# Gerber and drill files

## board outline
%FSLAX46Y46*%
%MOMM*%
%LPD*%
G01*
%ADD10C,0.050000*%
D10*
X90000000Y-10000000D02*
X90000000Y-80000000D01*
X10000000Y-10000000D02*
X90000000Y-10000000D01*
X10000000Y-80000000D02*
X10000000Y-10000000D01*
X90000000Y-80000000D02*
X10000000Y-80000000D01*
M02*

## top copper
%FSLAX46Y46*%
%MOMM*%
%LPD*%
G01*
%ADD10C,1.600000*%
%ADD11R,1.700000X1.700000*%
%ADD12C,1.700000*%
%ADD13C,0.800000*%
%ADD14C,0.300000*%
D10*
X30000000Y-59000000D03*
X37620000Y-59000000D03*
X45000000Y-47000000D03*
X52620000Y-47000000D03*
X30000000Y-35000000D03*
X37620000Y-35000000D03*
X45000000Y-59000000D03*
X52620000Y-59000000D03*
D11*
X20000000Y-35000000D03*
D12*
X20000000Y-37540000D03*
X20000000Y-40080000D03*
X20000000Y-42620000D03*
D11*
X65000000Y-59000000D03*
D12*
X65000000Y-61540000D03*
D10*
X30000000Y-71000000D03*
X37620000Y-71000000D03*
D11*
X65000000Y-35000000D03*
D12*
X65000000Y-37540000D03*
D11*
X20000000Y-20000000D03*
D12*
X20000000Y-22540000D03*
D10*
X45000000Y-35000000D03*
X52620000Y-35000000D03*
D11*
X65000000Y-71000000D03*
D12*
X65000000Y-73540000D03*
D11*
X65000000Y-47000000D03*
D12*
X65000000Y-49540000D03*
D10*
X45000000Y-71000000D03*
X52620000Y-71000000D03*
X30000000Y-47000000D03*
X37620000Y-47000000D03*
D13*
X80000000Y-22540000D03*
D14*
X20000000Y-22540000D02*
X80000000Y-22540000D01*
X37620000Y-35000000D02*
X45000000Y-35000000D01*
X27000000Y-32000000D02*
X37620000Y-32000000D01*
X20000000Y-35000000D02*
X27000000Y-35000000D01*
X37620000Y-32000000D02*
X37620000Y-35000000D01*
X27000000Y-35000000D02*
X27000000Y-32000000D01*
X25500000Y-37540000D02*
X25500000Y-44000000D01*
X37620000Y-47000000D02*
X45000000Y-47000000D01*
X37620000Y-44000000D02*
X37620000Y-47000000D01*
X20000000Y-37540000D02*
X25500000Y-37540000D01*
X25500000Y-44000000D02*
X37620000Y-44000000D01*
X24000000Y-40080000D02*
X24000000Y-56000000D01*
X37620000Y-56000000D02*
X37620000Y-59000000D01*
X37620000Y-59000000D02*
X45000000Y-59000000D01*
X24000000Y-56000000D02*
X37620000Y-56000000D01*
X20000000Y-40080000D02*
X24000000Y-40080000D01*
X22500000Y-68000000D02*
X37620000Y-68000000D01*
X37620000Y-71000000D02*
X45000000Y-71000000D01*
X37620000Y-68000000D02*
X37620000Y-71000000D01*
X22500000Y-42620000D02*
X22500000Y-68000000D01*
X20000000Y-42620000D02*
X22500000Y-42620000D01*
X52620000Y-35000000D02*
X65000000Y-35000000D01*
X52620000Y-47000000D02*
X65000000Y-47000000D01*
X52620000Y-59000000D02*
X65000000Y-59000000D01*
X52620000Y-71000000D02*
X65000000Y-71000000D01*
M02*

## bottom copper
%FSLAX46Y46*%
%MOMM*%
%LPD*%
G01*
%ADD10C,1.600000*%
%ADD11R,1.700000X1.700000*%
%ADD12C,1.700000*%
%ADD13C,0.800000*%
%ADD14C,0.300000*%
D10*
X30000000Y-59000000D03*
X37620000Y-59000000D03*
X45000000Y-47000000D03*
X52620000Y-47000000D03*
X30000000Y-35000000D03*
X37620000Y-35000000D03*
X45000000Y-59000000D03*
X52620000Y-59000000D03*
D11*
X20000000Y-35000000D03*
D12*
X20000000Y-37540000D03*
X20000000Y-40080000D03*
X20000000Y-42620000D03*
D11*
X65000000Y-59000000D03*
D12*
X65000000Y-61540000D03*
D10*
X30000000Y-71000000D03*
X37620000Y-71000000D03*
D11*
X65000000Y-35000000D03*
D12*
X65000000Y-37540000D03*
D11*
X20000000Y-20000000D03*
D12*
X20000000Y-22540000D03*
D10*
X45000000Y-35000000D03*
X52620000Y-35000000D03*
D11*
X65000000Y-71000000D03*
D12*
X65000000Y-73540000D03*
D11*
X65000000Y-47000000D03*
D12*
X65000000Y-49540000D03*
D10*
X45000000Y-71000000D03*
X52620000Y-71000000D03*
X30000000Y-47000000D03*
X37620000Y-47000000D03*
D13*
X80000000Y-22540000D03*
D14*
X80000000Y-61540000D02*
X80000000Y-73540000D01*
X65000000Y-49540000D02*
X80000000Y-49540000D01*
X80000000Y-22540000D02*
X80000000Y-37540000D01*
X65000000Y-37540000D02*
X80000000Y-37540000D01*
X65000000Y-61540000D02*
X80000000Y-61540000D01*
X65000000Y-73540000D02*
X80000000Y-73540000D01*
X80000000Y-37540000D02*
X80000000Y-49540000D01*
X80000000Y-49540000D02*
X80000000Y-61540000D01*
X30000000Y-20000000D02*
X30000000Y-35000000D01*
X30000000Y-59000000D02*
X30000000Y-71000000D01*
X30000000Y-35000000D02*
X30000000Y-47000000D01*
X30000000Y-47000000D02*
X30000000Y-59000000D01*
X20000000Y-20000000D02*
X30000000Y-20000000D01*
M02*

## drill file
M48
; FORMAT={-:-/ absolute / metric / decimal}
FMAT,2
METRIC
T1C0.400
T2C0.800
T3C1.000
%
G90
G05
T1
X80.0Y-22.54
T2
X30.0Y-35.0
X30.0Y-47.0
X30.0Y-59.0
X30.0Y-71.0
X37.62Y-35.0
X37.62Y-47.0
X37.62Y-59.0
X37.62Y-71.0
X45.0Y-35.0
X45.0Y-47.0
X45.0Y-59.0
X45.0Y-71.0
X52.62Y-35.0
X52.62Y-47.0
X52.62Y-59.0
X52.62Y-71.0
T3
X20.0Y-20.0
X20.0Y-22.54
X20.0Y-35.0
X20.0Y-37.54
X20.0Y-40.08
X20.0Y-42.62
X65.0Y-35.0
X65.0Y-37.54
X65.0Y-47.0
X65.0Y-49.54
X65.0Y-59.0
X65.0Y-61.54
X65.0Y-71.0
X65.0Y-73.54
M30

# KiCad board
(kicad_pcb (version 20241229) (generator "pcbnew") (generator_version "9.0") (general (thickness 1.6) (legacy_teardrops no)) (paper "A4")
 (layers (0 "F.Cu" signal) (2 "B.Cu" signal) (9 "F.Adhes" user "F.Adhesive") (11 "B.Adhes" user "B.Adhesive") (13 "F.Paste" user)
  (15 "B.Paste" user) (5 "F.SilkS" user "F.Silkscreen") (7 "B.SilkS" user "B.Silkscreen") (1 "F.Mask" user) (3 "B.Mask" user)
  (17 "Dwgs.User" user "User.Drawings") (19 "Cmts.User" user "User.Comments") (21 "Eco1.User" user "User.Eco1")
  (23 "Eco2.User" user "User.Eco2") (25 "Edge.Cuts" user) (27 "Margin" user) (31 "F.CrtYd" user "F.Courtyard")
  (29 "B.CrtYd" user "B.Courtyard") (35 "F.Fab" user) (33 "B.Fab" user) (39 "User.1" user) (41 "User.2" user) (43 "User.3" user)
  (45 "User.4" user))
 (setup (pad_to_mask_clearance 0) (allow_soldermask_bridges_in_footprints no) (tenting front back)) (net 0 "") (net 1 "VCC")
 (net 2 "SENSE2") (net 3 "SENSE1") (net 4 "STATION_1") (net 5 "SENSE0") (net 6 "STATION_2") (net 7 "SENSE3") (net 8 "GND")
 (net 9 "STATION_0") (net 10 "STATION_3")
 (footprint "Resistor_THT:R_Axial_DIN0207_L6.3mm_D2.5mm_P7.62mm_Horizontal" (layer "F.Cu") (at 30 59)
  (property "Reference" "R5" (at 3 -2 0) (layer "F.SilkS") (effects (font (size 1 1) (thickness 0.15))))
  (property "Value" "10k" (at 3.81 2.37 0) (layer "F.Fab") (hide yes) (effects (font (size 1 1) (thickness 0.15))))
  (pad "1" thru_hole circle (at 0 0) (size 1.6 1.6) (drill 0.8) (layers "*.Cu" "*.Mask") (remove_unused_layers no) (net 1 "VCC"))
  (pad "2" thru_hole circle (at 7.62 0) (size 1.6 1.6) (drill 0.8) (layers "*.Cu" "*.Mask") (remove_unused_layers no) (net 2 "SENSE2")))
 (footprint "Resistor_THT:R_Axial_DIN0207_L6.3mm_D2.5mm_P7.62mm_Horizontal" (layer "F.Cu") (at 45 47)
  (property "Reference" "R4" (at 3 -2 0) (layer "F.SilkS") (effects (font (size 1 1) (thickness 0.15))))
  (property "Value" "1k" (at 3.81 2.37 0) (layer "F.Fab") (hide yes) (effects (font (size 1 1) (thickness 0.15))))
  (pad "1" thru_hole circle (at 0 0) (size 1.6 1.6) (drill 0.8) (layers "*.Cu" "*.Mask") (remove_unused_layers no) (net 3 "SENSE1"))
  (pad "2" thru_hole circle (at 7.62 0) (size 1.6 1.6) (drill 0.8) (layers "*.Cu" "*.Mask") (remove_unused_layers no) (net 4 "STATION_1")))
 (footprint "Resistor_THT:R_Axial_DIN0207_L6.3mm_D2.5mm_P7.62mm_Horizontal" (layer "F.Cu") (at 30 35)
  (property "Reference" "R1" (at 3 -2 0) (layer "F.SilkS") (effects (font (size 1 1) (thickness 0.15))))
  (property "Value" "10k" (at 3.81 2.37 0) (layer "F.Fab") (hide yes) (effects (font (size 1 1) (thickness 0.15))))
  (pad "1" thru_hole circle (at 0 0) (size 1.6 1.6) (drill 0.8) (layers "*.Cu" "*.Mask") (remove_unused_layers no) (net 1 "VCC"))
  (pad "2" thru_hole circle (at 7.62 0) (size 1.6 1.6) (drill 0.8) (layers "*.Cu" "*.Mask") (remove_unused_layers no) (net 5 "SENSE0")))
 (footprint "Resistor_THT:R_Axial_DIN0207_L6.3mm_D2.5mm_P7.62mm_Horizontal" (layer "F.Cu") (at 45 59)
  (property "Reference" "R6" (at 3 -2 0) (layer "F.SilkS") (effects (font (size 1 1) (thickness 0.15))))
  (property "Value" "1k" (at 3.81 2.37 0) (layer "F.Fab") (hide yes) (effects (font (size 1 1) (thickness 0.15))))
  (pad "1" thru_hole circle (at 0 0) (size 1.6 1.6) (drill 0.8) (layers "*.Cu" "*.Mask") (remove_unused_layers no) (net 2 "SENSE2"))
  (pad "2" thru_hole circle (at 7.62 0) (size 1.6 1.6) (drill 0.8) (layers "*.Cu" "*.Mask") (remove_unused_layers no) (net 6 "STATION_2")))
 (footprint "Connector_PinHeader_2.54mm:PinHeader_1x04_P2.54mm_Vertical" (layer "F.Cu") (at 20 35)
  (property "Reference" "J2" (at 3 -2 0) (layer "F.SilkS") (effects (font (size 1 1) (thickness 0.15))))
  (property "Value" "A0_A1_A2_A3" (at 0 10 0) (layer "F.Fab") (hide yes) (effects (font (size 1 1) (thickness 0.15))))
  (pad "1" thru_hole rect (at 0 0) (size 1.7 1.7) (drill 1) (layers "*.Cu" "*.Mask") (remove_unused_layers no) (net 5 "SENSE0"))
  (pad "2" thru_hole circle (at 0 2.54) (size 1.7 1.7) (drill 1) (layers "*.Cu" "*.Mask") (remove_unused_layers no) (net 3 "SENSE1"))
  (pad "3" thru_hole circle (at 0 5.08) (size 1.7 1.7) (drill 1) (layers "*.Cu" "*.Mask") (remove_unused_layers no) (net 2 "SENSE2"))
  (pad "4" thru_hole circle (at 0 7.62) (size 1.7 1.7) (drill 1) (layers "*.Cu" "*.Mask") (remove_unused_layers no) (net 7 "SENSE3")))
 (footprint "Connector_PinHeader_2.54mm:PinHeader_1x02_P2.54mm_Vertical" (layer "F.Cu") (at 65 59)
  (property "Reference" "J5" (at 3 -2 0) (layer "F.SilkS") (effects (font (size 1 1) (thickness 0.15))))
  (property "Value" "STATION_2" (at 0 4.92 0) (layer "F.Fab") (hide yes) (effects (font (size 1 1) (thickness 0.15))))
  (pad "1" thru_hole rect (at 0 0) (size 1.7 1.7) (drill 1) (layers "*.Cu" "*.Mask") (remove_unused_layers no) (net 6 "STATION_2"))
  (pad "2" thru_hole circle (at 0 2.54) (size 1.7 1.7) (drill 1) (layers "*.Cu" "*.Mask") (remove_unused_layers no) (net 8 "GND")))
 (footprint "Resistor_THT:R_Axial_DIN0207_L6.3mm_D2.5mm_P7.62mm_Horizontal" (layer "F.Cu") (at 30 71)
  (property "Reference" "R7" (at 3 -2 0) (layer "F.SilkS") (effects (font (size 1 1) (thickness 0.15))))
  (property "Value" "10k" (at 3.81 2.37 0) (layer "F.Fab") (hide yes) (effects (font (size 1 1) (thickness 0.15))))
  (pad "1" thru_hole circle (at 0 0) (size 1.6 1.6) (drill 0.8) (layers "*.Cu" "*.Mask") (remove_unused_layers no) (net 1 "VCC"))
  (pad "2" thru_hole circle (at 7.62 0) (size 1.6 1.6) (drill 0.8) (layers "*.Cu" "*.Mask") (remove_unused_layers no) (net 7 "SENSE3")))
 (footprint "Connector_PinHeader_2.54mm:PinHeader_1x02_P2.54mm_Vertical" (layer "F.Cu") (at 65 35)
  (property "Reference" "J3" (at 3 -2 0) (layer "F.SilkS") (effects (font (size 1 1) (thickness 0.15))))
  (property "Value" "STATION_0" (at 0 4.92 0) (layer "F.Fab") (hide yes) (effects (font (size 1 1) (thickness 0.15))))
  (pad "1" thru_hole rect (at 0 0) (size 1.7 1.7) (drill 1) (layers "*.Cu" "*.Mask") (remove_unused_layers no) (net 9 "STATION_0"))
  (pad "2" thru_hole circle (at 0 2.54) (size 1.7 1.7) (drill 1) (layers "*.Cu" "*.Mask") (remove_unused_layers no) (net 8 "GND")))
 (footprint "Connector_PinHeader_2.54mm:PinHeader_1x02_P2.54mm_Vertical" (layer "F.Cu") (at 20 20)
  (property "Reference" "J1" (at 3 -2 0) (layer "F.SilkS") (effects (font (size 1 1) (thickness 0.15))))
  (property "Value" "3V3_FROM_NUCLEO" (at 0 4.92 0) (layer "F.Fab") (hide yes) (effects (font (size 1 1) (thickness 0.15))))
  (pad "1" thru_hole rect (at 0 0) (size 1.7 1.7) (drill 1) (layers "*.Cu" "*.Mask") (remove_unused_layers no) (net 1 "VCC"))
  (pad "2" thru_hole circle (at 0 2.54) (size 1.7 1.7) (drill 1) (layers "*.Cu" "*.Mask") (remove_unused_layers no) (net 8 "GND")))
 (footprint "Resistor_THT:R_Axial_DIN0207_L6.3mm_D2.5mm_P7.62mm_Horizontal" (layer "F.Cu") (at 45 35)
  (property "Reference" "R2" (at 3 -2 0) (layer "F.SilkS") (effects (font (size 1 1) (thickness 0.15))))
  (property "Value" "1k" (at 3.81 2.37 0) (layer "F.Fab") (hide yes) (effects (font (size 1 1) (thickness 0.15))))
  (pad "1" thru_hole circle (at 0 0) (size 1.6 1.6) (drill 0.8) (layers "*.Cu" "*.Mask") (remove_unused_layers no) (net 5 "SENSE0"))
  (pad "2" thru_hole circle (at 7.62 0) (size 1.6 1.6) (drill 0.8) (layers "*.Cu" "*.Mask") (remove_unused_layers no) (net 9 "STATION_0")))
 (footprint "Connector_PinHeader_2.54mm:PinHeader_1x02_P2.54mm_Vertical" (layer "F.Cu") (at 65 71)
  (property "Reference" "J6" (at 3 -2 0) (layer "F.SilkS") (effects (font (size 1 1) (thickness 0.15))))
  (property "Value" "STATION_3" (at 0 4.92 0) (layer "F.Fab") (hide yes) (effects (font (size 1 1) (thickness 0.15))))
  (pad "1" thru_hole rect (at 0 0) (size 1.7 1.7) (drill 1) (layers "*.Cu" "*.Mask") (remove_unused_layers no) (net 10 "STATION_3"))
  (pad "2" thru_hole circle (at 0 2.54) (size 1.7 1.7) (drill 1) (layers "*.Cu" "*.Mask") (remove_unused_layers no) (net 8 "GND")))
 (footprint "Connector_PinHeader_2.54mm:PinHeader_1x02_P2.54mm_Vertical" (layer "F.Cu") (at 65 47)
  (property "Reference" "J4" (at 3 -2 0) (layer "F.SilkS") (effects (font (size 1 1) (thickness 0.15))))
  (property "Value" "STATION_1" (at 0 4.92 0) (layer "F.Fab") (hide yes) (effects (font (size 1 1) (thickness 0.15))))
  (pad "1" thru_hole rect (at 0 0) (size 1.7 1.7) (drill 1) (layers "*.Cu" "*.Mask") (remove_unused_layers no) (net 4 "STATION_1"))
  (pad "2" thru_hole circle (at 0 2.54) (size 1.7 1.7) (drill 1) (layers "*.Cu" "*.Mask") (remove_unused_layers no) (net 8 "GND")))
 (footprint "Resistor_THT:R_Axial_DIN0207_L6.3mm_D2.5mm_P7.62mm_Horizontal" (layer "F.Cu") (at 45 71)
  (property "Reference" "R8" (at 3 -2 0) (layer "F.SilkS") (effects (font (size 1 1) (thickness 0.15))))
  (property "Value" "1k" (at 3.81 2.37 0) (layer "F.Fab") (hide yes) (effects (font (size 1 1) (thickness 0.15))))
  (pad "1" thru_hole circle (at 0 0) (size 1.6 1.6) (drill 0.8) (layers "*.Cu" "*.Mask") (remove_unused_layers no) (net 7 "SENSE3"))
  (pad "2" thru_hole circle (at 7.62 0) (size 1.6 1.6) (drill 0.8) (layers "*.Cu" "*.Mask") (remove_unused_layers no) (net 10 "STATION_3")))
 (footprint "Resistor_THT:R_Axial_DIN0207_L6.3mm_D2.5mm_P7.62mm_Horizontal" (layer "F.Cu") (at 30 47)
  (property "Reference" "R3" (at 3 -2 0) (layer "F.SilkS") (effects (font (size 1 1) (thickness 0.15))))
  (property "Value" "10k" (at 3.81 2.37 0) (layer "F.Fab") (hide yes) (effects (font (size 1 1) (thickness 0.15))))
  (pad "1" thru_hole circle (at 0 0) (size 1.6 1.6) (drill 0.8) (layers "*.Cu" "*.Mask") (remove_unused_layers no) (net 1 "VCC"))
  (pad "2" thru_hole circle (at 7.62 0) (size 1.6 1.6) (drill 0.8) (layers "*.Cu" "*.Mask") (remove_unused_layers no) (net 3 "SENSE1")))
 (gr_line (start 90 10) (end 90 80) (stroke (width 0.05) (type default)) (layer "Edge.Cuts"))
 (gr_line (start 10 10) (end 90 10) (stroke (width 0.05) (type default)) (layer "Edge.Cuts"))
 (gr_line (start 10 80) (end 10 10) (stroke (width 0.05) (type default)) (layer "Edge.Cuts"))
 (gr_line (start 90 80) (end 10 80) (stroke (width 0.05) (type default)) (layer "Edge.Cuts"))
 (segment (start 20 22.54) (end 80 22.54) (width 0.3) (layer "F.Cu") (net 8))
 (via (at 80 22.54) (size 0.8) (drill 0.4) (layers "F.Cu" "B.Cu") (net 8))
 (segment (start 80 61.54) (end 80 73.54) (width 0.3) (layer "B.Cu") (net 8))
 (segment (start 65 49.54) (end 80 49.54) (width 0.3) (layer "B.Cu") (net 8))
 (segment (start 80 22.54) (end 80 37.54) (width 0.3) (layer "B.Cu") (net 8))
 (segment (start 65 37.54) (end 80 37.54) (width 0.3) (layer "B.Cu") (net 8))
 (segment (start 65 61.54) (end 80 61.54) (width 0.3) (layer "B.Cu") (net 8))
 (segment (start 65 73.54) (end 80 73.54) (width 0.3) (layer "B.Cu") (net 8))
 (segment (start 80 37.54) (end 80 49.54) (width 0.3) (layer "B.Cu") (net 8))
 (segment (start 80 49.54) (end 80 61.54) (width 0.3) (layer "B.Cu") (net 8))
 (segment (start 37.62 35) (end 45 35) (width 0.3) (layer "F.Cu") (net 5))
 (segment (start 27 32) (end 37.62 32) (width 0.3) (layer "F.Cu") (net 5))
 (segment (start 20 35) (end 27 35) (width 0.3) (layer "F.Cu") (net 5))
 (segment (start 37.62 32) (end 37.62 35) (width 0.3) (layer "F.Cu") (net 5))
 (segment (start 27 35) (end 27 32) (width 0.3) (layer "F.Cu") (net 5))
 (segment (start 25.5 37.54) (end 25.5 44) (width 0.3) (layer "F.Cu") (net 3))
 (segment (start 37.62 47) (end 45 47) (width 0.3) (layer "F.Cu") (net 3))
 (segment (start 37.62 44) (end 37.62 47) (width 0.3) (layer "F.Cu") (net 3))
 (segment (start 20 37.54) (end 25.5 37.54) (width 0.3) (layer "F.Cu") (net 3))
 (segment (start 25.5 44) (end 37.62 44) (width 0.3) (layer "F.Cu") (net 3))
 (segment (start 24 40.08) (end 24 56) (width 0.3) (layer "F.Cu") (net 2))
 (segment (start 37.62 56) (end 37.62 59) (width 0.3) (layer "F.Cu") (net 2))
 (segment (start 37.62 59) (end 45 59) (width 0.3) (layer "F.Cu") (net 2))
 (segment (start 24 56) (end 37.62 56) (width 0.3) (layer "F.Cu") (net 2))
 (segment (start 20 40.08) (end 24 40.08) (width 0.3) (layer "F.Cu") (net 2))
 (segment (start 22.5 68) (end 37.62 68) (width 0.3) (layer "F.Cu") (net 7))
 (segment (start 37.62 71) (end 45 71) (width 0.3) (layer "F.Cu") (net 7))
 (segment (start 37.62 68) (end 37.62 71) (width 0.3) (layer "F.Cu") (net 7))
 (segment (start 22.5 42.62) (end 22.5 68) (width 0.3) (layer "F.Cu") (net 7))
 (segment (start 20 42.62) (end 22.5 42.62) (width 0.3) (layer "F.Cu") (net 7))
 (segment (start 52.62 35) (end 65 35) (width 0.3) (layer "F.Cu") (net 9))
 (segment (start 52.62 47) (end 65 47) (width 0.3) (layer "F.Cu") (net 4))
 (segment (start 52.62 59) (end 65 59) (width 0.3) (layer "F.Cu") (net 6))
 (segment (start 52.62 71) (end 65 71) (width 0.3) (layer "F.Cu") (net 10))
 (segment (start 30 20) (end 30 35) (width 0.3) (layer "B.Cu") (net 1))
 (segment (start 30 59) (end 30 71) (width 0.3) (layer "B.Cu") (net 1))
 (segment (start 30 35) (end 30 47) (width 0.3) (layer "B.Cu") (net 1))
 (segment (start 30 47) (end 30 59) (width 0.3) (layer "B.Cu") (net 1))
 (segment (start 20 20) (end 30 20) (width 0.3) (layer "B.Cu") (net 1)))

